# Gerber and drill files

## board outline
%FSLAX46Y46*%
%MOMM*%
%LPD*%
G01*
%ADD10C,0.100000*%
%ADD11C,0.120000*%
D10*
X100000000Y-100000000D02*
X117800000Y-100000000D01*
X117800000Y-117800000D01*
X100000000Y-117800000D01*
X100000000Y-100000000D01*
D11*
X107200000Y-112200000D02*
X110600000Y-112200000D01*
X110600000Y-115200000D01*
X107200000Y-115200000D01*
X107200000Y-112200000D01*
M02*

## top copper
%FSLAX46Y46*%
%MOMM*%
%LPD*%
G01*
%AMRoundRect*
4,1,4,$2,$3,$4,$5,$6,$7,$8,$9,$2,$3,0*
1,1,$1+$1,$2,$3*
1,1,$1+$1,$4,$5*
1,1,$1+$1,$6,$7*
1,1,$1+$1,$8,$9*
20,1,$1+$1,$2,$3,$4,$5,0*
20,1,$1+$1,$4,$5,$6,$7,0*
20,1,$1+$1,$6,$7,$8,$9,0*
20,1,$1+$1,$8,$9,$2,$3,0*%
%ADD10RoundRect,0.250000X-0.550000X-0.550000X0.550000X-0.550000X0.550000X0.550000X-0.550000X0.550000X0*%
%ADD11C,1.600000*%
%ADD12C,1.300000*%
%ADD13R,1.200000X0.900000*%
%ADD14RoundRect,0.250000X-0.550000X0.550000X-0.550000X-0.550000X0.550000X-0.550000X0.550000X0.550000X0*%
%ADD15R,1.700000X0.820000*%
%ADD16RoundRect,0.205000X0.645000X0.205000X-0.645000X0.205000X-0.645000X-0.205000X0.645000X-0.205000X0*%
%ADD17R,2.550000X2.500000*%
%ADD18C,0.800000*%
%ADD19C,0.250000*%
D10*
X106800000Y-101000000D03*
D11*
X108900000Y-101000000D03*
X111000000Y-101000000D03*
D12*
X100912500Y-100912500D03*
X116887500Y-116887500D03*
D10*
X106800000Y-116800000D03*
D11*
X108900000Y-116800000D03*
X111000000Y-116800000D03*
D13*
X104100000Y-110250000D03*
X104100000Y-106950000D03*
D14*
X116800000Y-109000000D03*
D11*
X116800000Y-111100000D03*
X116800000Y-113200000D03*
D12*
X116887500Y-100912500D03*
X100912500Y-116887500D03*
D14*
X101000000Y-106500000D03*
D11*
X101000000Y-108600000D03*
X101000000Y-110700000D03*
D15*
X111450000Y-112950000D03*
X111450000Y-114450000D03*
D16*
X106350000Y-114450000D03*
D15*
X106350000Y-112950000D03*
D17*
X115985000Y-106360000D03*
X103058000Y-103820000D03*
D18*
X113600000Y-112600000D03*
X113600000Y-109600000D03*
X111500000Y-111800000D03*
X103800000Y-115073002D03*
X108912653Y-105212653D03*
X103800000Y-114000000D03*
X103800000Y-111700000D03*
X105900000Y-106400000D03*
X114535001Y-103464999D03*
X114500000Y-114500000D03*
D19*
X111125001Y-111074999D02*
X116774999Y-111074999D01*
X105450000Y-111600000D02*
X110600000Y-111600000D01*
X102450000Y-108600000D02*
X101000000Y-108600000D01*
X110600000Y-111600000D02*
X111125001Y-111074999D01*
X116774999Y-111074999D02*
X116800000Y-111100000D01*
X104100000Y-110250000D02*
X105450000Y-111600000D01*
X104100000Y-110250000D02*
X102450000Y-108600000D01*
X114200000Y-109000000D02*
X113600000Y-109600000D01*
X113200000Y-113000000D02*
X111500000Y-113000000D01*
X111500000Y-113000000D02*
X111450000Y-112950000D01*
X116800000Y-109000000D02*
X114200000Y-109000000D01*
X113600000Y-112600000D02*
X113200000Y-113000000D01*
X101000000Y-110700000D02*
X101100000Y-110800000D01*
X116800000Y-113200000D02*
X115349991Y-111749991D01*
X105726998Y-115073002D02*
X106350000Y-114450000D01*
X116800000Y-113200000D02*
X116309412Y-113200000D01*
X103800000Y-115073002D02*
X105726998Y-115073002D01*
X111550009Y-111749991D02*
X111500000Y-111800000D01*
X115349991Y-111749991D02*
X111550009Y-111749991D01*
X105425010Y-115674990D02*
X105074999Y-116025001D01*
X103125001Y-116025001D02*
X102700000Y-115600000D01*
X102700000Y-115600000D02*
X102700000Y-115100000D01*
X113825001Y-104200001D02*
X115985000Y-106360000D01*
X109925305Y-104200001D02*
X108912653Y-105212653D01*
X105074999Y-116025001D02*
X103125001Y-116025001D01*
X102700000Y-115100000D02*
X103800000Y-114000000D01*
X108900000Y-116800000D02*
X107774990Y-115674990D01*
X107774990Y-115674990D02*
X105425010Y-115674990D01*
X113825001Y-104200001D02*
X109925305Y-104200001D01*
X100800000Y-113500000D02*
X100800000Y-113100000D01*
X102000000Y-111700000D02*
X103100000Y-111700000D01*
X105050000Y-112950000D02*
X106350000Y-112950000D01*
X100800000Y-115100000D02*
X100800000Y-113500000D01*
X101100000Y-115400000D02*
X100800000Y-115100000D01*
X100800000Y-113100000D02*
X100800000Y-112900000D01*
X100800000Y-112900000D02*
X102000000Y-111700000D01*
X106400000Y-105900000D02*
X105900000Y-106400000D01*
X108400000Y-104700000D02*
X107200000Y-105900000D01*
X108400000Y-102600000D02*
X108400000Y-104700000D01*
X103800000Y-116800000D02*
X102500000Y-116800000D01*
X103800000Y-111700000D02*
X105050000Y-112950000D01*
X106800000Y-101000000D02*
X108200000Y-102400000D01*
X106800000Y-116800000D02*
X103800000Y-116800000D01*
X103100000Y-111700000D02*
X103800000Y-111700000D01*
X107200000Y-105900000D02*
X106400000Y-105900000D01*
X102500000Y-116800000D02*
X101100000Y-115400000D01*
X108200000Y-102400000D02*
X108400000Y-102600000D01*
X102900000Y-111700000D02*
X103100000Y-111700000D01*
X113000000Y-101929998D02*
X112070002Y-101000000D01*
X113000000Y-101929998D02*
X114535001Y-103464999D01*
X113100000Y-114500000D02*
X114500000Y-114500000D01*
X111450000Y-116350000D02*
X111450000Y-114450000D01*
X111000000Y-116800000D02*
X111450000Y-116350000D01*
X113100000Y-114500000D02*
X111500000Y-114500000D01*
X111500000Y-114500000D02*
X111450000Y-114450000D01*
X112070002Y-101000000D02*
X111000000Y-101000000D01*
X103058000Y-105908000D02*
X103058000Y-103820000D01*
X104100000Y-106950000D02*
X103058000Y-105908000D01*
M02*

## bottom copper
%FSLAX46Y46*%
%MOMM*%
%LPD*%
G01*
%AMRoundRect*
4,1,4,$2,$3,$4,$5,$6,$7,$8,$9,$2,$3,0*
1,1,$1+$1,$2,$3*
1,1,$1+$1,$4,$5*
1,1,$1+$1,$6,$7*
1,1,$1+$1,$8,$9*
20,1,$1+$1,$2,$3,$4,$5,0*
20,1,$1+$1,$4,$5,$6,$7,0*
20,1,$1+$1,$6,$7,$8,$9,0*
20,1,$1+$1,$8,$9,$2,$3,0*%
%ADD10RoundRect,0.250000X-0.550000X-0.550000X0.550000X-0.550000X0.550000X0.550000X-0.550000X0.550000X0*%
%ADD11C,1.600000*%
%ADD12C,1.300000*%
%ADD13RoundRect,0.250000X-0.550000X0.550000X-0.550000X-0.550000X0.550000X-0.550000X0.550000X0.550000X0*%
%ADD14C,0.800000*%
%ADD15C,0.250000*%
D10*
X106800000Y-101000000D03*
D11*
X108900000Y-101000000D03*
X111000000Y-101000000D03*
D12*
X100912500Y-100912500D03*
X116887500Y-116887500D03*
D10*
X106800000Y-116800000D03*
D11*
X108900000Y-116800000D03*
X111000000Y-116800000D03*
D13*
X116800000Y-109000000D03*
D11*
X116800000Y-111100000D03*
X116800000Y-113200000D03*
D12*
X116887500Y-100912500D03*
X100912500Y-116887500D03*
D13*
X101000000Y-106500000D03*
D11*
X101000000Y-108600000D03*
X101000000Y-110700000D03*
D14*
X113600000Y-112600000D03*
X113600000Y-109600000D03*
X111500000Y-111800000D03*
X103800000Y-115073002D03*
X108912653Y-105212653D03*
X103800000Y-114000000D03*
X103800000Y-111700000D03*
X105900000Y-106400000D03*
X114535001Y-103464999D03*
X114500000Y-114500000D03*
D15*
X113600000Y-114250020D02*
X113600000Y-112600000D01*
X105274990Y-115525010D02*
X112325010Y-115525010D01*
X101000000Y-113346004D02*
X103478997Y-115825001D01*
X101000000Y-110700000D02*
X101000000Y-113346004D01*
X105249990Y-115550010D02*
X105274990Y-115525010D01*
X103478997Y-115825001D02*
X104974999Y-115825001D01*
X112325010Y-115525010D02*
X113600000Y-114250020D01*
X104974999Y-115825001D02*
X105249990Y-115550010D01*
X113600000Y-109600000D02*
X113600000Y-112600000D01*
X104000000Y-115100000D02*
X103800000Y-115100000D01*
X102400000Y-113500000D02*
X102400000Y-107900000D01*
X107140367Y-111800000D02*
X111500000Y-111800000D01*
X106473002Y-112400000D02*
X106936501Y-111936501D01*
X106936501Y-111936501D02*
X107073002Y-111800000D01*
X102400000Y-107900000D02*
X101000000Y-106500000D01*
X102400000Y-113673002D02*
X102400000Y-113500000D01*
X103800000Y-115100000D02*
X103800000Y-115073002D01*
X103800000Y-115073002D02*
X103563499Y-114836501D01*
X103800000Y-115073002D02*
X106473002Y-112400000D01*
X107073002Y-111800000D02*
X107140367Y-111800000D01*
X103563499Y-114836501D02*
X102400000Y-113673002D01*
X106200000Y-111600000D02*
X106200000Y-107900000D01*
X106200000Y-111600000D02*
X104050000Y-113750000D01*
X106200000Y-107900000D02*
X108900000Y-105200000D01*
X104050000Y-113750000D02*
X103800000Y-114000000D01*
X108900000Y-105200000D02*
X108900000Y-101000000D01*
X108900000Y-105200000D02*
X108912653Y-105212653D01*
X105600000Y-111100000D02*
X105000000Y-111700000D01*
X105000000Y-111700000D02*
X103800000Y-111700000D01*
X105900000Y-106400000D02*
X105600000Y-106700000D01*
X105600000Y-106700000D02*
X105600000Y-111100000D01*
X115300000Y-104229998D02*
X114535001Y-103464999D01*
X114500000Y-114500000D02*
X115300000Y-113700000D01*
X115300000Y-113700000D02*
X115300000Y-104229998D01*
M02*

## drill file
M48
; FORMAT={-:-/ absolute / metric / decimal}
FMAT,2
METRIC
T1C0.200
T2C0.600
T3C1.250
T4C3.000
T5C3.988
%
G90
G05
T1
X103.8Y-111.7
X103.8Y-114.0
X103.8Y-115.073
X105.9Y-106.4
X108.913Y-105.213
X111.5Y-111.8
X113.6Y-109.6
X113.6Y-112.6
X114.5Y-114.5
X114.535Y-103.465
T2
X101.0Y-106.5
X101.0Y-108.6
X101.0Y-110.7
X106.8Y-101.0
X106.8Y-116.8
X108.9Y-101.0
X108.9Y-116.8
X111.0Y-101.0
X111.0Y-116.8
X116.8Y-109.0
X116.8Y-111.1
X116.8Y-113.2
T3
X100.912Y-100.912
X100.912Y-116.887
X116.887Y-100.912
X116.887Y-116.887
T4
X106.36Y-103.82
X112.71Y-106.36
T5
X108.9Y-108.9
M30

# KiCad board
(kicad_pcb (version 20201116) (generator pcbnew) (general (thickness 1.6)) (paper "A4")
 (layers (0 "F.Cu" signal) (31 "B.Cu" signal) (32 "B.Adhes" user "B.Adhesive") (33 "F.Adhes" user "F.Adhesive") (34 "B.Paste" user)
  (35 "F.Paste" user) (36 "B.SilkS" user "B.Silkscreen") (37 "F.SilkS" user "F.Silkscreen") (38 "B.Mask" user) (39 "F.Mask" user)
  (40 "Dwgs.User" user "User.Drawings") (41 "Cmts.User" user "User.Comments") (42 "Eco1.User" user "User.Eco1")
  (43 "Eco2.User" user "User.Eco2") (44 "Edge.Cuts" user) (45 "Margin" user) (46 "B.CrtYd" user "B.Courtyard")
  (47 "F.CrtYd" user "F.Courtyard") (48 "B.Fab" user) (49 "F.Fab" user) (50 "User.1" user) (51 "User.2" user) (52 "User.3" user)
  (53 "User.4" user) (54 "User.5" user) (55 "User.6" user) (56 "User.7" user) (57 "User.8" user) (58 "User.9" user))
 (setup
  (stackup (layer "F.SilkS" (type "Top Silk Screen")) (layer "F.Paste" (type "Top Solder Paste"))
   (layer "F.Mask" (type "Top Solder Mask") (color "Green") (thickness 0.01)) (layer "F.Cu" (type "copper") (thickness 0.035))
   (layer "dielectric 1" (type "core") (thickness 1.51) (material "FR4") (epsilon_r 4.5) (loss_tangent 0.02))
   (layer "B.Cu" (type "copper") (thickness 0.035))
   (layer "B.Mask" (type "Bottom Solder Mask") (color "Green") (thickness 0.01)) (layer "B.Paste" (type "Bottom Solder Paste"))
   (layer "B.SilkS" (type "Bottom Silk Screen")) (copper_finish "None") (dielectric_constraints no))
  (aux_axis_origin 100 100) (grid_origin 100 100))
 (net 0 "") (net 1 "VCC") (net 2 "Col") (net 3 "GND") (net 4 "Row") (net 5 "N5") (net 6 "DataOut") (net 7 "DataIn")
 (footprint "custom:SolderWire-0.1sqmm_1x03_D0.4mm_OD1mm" (layer "F.Cu") (at 106.8 101)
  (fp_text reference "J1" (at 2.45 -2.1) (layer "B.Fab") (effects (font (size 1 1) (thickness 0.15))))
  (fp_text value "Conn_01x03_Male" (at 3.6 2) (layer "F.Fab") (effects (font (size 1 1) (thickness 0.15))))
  (pad "1" thru_hole roundrect (at 0 0) (size 1.6 1.6) (drill 0.6) (layers *.Cu *.Mask) (roundrect_rratio 0.15625) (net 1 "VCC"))
  (pad "2" thru_hole circle (at 2.1 0) (size 1.6 1.6) (drill 0.6) (layers *.Cu *.Mask) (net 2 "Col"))
  (pad "3" thru_hole circle (at 4.2 0) (size 1.6 1.6) (drill 0.6) (layers *.Cu *.Mask) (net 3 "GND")))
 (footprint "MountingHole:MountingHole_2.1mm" (layer "F.Cu") (at 100.9125 100.9125)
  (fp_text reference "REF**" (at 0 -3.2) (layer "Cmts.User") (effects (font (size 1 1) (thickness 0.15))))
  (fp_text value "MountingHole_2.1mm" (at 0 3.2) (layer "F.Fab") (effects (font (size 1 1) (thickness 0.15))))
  (pad "" np_thru_hole circle (at 0 0) (size 1.3 1.3) (drill 1.25) (layers F&B.Cu *.Mask)))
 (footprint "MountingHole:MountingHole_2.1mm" (layer "F.Cu") (at 116.8875 116.8875)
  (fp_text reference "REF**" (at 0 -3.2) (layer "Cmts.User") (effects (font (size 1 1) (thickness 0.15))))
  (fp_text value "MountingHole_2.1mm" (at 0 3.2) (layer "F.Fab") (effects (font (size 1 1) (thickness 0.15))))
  (pad "" np_thru_hole circle (at 0 0) (size 1.3 1.3) (drill 1.25) (layers F&B.Cu *.Mask)))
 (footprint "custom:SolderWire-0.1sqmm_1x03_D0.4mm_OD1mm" (layer "F.Cu") (at 106.8 116.8)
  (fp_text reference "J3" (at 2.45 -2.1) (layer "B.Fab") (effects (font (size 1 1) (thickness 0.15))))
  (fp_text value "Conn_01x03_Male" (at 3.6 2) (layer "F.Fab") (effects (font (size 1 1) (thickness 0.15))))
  (pad "1" thru_hole roundrect (at 0 0) (size 1.6 1.6) (drill 0.6) (layers *.Cu *.Mask) (roundrect_rratio 0.15625) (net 1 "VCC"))
  (pad "2" thru_hole circle (at 2.1 0) (size 1.6 1.6) (drill 0.6) (layers *.Cu *.Mask) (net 2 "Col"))
  (pad "3" thru_hole circle (at 4.2 0) (size 1.6 1.6) (drill 0.6) (layers *.Cu *.Mask) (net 3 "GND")))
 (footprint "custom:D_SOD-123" (layer "F.Cu") (at 104.1 108.6 90)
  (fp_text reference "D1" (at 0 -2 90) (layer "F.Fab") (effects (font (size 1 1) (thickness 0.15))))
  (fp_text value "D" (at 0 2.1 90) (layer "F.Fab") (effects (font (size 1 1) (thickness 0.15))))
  (pad "1" smd rect (at -1.65 0 90) (size 0.9 1.2) (layers "F.Cu" "F.Paste" "F.Mask") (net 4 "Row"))
  (pad "2" smd rect (at 1.65 0 90) (size 0.9 1.2) (layers "F.Cu" "F.Paste" "F.Mask") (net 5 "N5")))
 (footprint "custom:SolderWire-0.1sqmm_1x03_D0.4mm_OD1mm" (layer "F.Cu") (at 116.8 109 -90)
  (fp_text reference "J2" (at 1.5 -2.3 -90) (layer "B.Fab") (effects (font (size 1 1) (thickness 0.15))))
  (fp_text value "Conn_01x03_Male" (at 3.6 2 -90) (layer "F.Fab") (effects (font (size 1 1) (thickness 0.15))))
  (pad "1" thru_hole roundrect (at 0 0 270) (size 1.6 1.6) (drill 0.6) (layers *.Cu *.Mask) (roundrect_rratio 0.15625) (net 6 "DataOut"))
  (pad "2" thru_hole circle (at 2.1 0 270) (size 1.6 1.6) (drill 0.6) (layers *.Cu *.Mask) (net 4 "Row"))
  (pad "3" thru_hole circle (at 4.2 0 270) (size 1.6 1.6) (drill 0.6) (layers *.Cu *.Mask) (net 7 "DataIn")))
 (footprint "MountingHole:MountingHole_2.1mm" (layer "F.Cu") (at 116.8875 100.9125)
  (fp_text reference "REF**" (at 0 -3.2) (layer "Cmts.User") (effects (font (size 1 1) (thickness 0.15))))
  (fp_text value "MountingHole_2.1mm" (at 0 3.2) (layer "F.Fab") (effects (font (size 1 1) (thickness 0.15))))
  (pad "" np_thru_hole circle (at 0 0) (size 1.3 1.3) (drill 1.25) (layers F&B.Cu *.Mask)))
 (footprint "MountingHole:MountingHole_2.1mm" (layer "F.Cu") (at 100.9125 116.8875)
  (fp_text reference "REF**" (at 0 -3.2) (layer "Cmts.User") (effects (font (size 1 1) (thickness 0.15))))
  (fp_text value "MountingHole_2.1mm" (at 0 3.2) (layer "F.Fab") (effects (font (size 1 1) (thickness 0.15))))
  (pad "" np_thru_hole circle (at 0 0) (size 1.3 1.3) (drill 1.25) (layers F&B.Cu *.Mask)))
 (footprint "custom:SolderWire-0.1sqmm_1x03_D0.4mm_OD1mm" (layer "F.Cu") (at 101 106.5 -90)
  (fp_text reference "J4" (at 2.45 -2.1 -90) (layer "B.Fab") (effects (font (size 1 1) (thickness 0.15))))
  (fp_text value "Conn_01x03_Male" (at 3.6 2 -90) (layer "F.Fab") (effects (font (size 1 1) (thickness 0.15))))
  (pad "1" thru_hole roundrect (at 0 0 270) (size 1.6 1.6) (drill 0.6) (layers *.Cu *.Mask) (roundrect_rratio 0.15625) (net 7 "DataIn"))
  (pad "2" thru_hole circle (at 2.1 0 270) (size 1.6 1.6) (drill 0.6) (layers *.Cu *.Mask) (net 4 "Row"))
  (pad "3" thru_hole circle (at 4.2 0 270) (size 1.6 1.6) (drill 0.6) (layers *.Cu *.Mask) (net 6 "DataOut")))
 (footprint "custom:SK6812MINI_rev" (layer "F.Cu") (at 108.9 113.7 180)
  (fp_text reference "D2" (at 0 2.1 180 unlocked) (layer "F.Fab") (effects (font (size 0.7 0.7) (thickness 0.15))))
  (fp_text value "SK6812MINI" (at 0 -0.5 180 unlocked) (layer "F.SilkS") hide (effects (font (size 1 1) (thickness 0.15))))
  (fp_rect (start 1.7 -1.5) (end -1.7 1.5) (layer "Edge.Cuts") (width 0.12) (fill none))
  (pad "1" smd rect (at -2.55 0.75 180) (size 1.7 0.82) (layers "F.Cu" "F.Paste" "F.Mask") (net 6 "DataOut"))
  (pad "2" smd rect (at -2.55 -0.75 180) (size 1.7 0.82) (layers "F.Cu" "F.Paste" "F.Mask") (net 3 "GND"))
  (pad "3" smd roundrect (at 2.55 -0.75 180) (size 1.7 0.82) (layers "F.Cu" "F.Paste" "F.Mask") (roundrect_rratio 0.25) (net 7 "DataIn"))
  (pad "4" smd rect (at 2.55 0.75 180) (size 1.7 0.82) (layers "F.Cu" "F.Paste" "F.Mask") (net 1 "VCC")))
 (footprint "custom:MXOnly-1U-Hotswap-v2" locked (layer "B.Cu") (at 108.9 108.9 180)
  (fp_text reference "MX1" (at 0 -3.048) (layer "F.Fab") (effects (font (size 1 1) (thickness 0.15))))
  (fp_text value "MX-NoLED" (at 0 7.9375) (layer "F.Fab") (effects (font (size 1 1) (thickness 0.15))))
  (pad "" np_thru_hole circle (at 0 0 180) (size 3.9878 3.9878) (drill 3.9878) (layers *.Cu *.Mask))
  (pad "" np_thru_hole circle (at 2.54 5.08 180) (size 3 3) (drill 3) (layers *.Cu *.Mask))
  (pad "" np_thru_hole circle (at -3.81 2.54 180) (size 3 3) (drill 3) (layers *.Cu *.Mask))
  (pad "1" smd rect (at -7.085 2.54 180) (size 2.55 2.5) (layers "F.Cu" "F.Paste" "F.Mask") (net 2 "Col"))
  (pad "2" smd rect (at 5.842 5.08 180) (size 2.55 2.5) (layers "F.Cu" "F.Paste" "F.Mask") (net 5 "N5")))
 (gr_rect (start 100 100) (end 117.8 117.8) (layer "Edge.Cuts") (width 0.1) (fill none))
 (segment (start 111.125001 111.074999) (end 116.774999 111.074999) (width 0.25) (layer "F.Cu") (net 4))
 (segment (start 105.45 111.6) (end 110.6 111.6) (width 0.25) (layer "F.Cu") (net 4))
 (segment (start 102.45 108.6) (end 101 108.6) (width 0.25) (layer "F.Cu") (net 4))
 (segment (start 110.6 111.6) (end 111.125001 111.074999) (width 0.25) (layer "F.Cu") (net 4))
 (segment (start 116.774999 111.074999) (end 116.8 111.1) (width 0.25) (layer "F.Cu") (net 4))
 (segment (start 104.1 110.25) (end 105.45 111.6) (width 0.25) (layer "F.Cu") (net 4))
 (segment (start 104.1 110.25) (end 102.45 108.6) (width 0.25) (layer "F.Cu") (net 4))
 (segment (start 114.2 109) (end 113.6 109.6) (width 0.25) (layer "F.Cu") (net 6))
 (segment (start 113.2 113) (end 111.5 113) (width 0.25) (layer "F.Cu") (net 6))
 (segment (start 111.5 113) (end 111.45 112.95) (width 0.25) (layer "F.Cu") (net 6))
 (segment (start 116.8 109) (end 114.2 109) (width 0.25) (layer "F.Cu") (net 6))
 (segment (start 113.6 112.6) (end 113.2 113) (width 0.25) (layer "F.Cu") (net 6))
 (segment (start 101 110.7) (end 101.1 110.8) (width 0.25) (layer "F.Cu") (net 6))
 (via (at 113.6 112.6) (size 0.8) (drill 0.2) (layers "F.Cu" "B.Cu") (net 6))
 (via (at 113.6 109.6) (size 0.8) (drill 0.2) (layers "F.Cu" "B.Cu") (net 6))
 (segment (start 113.6 114.25002) (end 113.6 112.6) (width 0.25) (layer "B.Cu") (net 6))
 (segment (start 105.27499 115.52501) (end 112.32501 115.52501) (width 0.25) (layer "B.Cu") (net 6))
 (segment (start 101 113.346004) (end 103.478997 115.825001) (width 0.25) (layer "B.Cu") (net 6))
 (segment (start 101 110.7) (end 101 113.346004) (width 0.25) (layer "B.Cu") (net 6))
 (segment (start 105.24999 115.55001) (end 105.27499 115.52501) (width 0.25) (layer "B.Cu") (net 6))
 (segment (start 103.478997 115.825001) (end 104.974999 115.825001) (width 0.25) (layer "B.Cu") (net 6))
 (segment (start 112.32501 115.52501) (end 113.6 114.25002) (width 0.25) (layer "B.Cu") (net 6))
 (segment (start 104.974999 115.825001) (end 105.24999 115.55001) (width 0.25) (layer "B.Cu") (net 6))
 (segment (start 113.6 109.6) (end 113.6 112.6) (width 0.25) (layer "B.Cu") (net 6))
 (segment (start 116.8 113.2) (end 115.349991 111.749991) (width 0.25) (layer "F.Cu") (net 7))
 (segment (start 105.726998 115.073002) (end 106.35 114.45) (width 0.25) (layer "F.Cu") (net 7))
 (segment (start 116.8 113.2) (end 116.309412 113.2) (width 0.25) (layer "F.Cu") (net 7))
 (segment (start 103.8 115.073002) (end 105.726998 115.073002) (width 0.25) (layer "F.Cu") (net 7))
 (segment (start 111.550009 111.749991) (end 111.5 111.8) (width 0.25) (layer "F.Cu") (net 7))
 (segment (start 115.349991 111.749991) (end 111.550009 111.749991) (width 0.25) (layer "F.Cu") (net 7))
 (via (at 111.5 111.8) (size 0.8) (drill 0.2) (layers "F.Cu" "B.Cu") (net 7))
 (via (at 103.8 115.073002) (size 0.8) (drill 0.2) (layers "F.Cu" "B.Cu") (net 7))
 (segment (start 104 115.1) (end 103.8 115.1) (width 0.25) (layer "B.Cu") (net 7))
 (segment (start 102.4 113.5) (end 102.4 107.9) (width 0.25) (layer "B.Cu") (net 7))
 (segment (start 107.140367 111.8) (end 111.5 111.8) (width 0.25) (layer "B.Cu") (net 7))
 (segment (start 106.473002 112.4) (end 106.936501 111.936501) (width 0.25) (layer "B.Cu") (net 7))
 (segment (start 106.936501 111.936501) (end 107.073002 111.8) (width 0.25) (layer "B.Cu") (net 7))
 (segment (start 102.4 107.9) (end 101 106.5) (width 0.25) (layer "B.Cu") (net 7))
 (segment (start 102.4 113.673002) (end 102.4 113.5) (width 0.25) (layer "B.Cu") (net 7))
 (segment (start 103.8 115.1) (end 103.8 115.073002) (width 0.25) (layer "B.Cu") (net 7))
 (segment (start 103.8 115.073002) (end 103.563499 114.836501) (width 0.25) (layer "B.Cu") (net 7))
 (segment (start 103.8 115.073002) (end 106.473002 112.4) (width 0.25) (layer "B.Cu") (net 7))
 (segment (start 107.073002 111.8) (end 107.140367 111.8) (width 0.25) (layer "B.Cu") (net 7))
 (segment (start 103.563499 114.836501) (end 102.4 113.673002) (width 0.25) (layer "B.Cu") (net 7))
 (segment (start 105.42501 115.67499) (end 105.074999 116.025001) (width 0.25) (layer "F.Cu") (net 2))
 (segment (start 103.125001 116.025001) (end 102.7 115.6) (width 0.25) (layer "F.Cu") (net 2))
 (segment (start 102.7 115.6) (end 102.7 115.1) (width 0.25) (layer "F.Cu") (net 2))
 (segment (start 113.825001 104.200001) (end 115.985 106.36) (width 0.25) (layer "F.Cu") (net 2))
 (segment (start 109.925305 104.200001) (end 108.912653 105.212653) (width 0.25) (layer "F.Cu") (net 2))
 (segment (start 105.074999 116.025001) (end 103.125001 116.025001) (width 0.25) (layer "F.Cu") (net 2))
 (segment (start 102.7 115.1) (end 103.8 114) (width 0.25) (layer "F.Cu") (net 2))
 (segment (start 108.9 116.8) (end 107.77499 115.67499) (width 0.25) (layer "F.Cu") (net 2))
 (segment (start 107.77499 115.67499) (end 105.42501 115.67499) (width 0.25) (layer "F.Cu") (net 2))
 (segment (start 113.825001 104.200001) (end 109.925305 104.200001) (width 0.25) (layer "F.Cu") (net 2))
 (via (at 108.912653 105.212653) (size 0.8) (drill 0.2) (layers "F.Cu" "B.Cu") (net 2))
 (via (at 103.8 114) (size 0.8) (drill 0.2) (layers "F.Cu" "B.Cu") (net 2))
 (segment (start 106.2 111.6) (end 106.2 107.9) (width 0.25) (layer "B.Cu") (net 2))
 (segment (start 106.2 111.6) (end 104.05 113.75) (width 0.25) (layer "B.Cu") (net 2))
 (segment (start 106.2 107.9) (end 108.9 105.2) (width 0.25) (layer "B.Cu") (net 2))
 (segment (start 104.05 113.75) (end 103.8 114) (width 0.25) (layer "B.Cu") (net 2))
 (segment (start 108.9 105.2) (end 108.9 101) (width 0.25) (layer "B.Cu") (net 2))
 (segment (start 108.9 105.2) (end 108.912653 105.212653) (width 0.25) (layer "B.Cu") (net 2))
 (segment (start 100.8 113.5) (end 100.8 113.1) (width 0.25) (layer "F.Cu") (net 1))
 (segment (start 102 111.7) (end 103.1 111.7) (width 0.25) (layer "F.Cu") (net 1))
 (segment (start 105.05 112.95) (end 106.35 112.95) (width 0.25) (layer "F.Cu") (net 1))
 (segment (start 100.8 115.1) (end 100.8 113.5) (width 0.25) (layer "F.Cu") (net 1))
 (segment (start 101.1 115.4) (end 100.8 115.1) (width 0.25) (layer "F.Cu") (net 1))
 (segment (start 100.8 113.1) (end 100.8 112.9) (width 0.25) (layer "F.Cu") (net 1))
 (segment (start 100.8 112.9) (end 102 111.7) (width 0.25) (layer "F.Cu") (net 1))
 (segment (start 106.4 105.9) (end 105.9 106.4) (width 0.25) (layer "F.Cu") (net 1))
 (segment (start 108.4 104.7) (end 107.2 105.9) (width 0.25) (layer "F.Cu") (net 1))
 (segment (start 108.4 102.6) (end 108.4 104.7) (width 0.25) (layer "F.Cu") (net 1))
 (segment (start 103.8 116.8) (end 102.5 116.8) (width 0.25) (layer "F.Cu") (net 1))
 (segment (start 103.8 111.7) (end 105.05 112.95) (width 0.25) (layer "F.Cu") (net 1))
 (segment (start 106.8 101) (end 108.2 102.4) (width 0.25) (layer "F.Cu") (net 1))
 (segment (start 106.8 116.8) (end 103.8 116.8) (width 0.25) (layer "F.Cu") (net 1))
 (segment (start 103.1 111.7) (end 103.8 111.7) (width 0.25) (layer "F.Cu") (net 1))
 (segment (start 107.2 105.9) (end 106.4 105.9) (width 0.25) (layer "F.Cu") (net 1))
 (segment (start 102.5 116.8) (end 101.1 115.4) (width 0.25) (layer "F.Cu") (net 1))
 (segment (start 108.2 102.4) (end 108.4 102.6) (width 0.25) (layer "F.Cu") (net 1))
 (segment (start 102.9 111.7) (end 103.1 111.7) (width 0.25) (layer "F.Cu") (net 1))
 (via (at 103.8 111.7) (size 0.8) (drill 0.2) (layers "F.Cu" "B.Cu") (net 1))
 (via (at 105.9 106.4) (size 0.8) (drill 0.2) (layers "F.Cu" "B.Cu") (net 1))
 (segment (start 105.6 111.1) (end 105 111.7) (width 0.25) (layer "B.Cu") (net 1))
 (segment (start 105 111.7) (end 103.8 111.7) (width 0.25) (layer "B.Cu") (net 1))
 (segment (start 105.9 106.4) (end 105.6 106.7) (width 0.25) (layer "B.Cu") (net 1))
 (segment (start 105.6 106.7) (end 105.6 111.1) (width 0.25) (layer "B.Cu") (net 1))
 (segment (start 113 101.929998) (end 112.070002 101) (width 0.25) (layer "F.Cu") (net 3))
 (segment (start 113 101.929998) (end 114.535001 103.464999) (width 0.25) (layer "F.Cu") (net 3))
 (segment (start 113.1 114.5) (end 114.5 114.5) (width 0.25) (layer "F.Cu") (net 3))
 (segment (start 111.45 116.35) (end 111.45 114.45) (width 0.25) (layer "F.Cu") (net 3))
 (segment (start 111 116.8) (end 111.45 116.35) (width 0.25) (layer "F.Cu") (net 3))
 (segment (start 113.1 114.5) (end 111.5 114.5) (width 0.25) (layer "F.Cu") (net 3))
 (segment (start 111.5 114.5) (end 111.45 114.45) (width 0.25) (layer "F.Cu") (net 3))
 (segment (start 112.070002 101) (end 111 101) (width 0.25) (layer "F.Cu") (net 3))
 (via (at 114.535001 103.464999) (size 0.8) (drill 0.2) (layers "F.Cu" "B.Cu") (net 3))
 (via (at 114.5 114.5) (size 0.8) (drill 0.2) (layers "F.Cu" "B.Cu") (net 3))
 (segment (start 115.3 104.229998) (end 114.535001 103.464999) (width 0.25) (layer "B.Cu") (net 3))
 (segment (start 114.5 114.5) (end 115.3 113.7) (width 0.25) (layer "B.Cu") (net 3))
 (segment (start 115.3 113.7) (end 115.3 104.229998) (width 0.25) (layer "B.Cu") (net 3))
 (segment (start 103.058 105.908) (end 103.058 103.82) (width 0.25) (layer "F.Cu") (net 5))
 (segment (start 104.1 106.95) (end 103.058 105.908) (width 0.25) (layer "F.Cu") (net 5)))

